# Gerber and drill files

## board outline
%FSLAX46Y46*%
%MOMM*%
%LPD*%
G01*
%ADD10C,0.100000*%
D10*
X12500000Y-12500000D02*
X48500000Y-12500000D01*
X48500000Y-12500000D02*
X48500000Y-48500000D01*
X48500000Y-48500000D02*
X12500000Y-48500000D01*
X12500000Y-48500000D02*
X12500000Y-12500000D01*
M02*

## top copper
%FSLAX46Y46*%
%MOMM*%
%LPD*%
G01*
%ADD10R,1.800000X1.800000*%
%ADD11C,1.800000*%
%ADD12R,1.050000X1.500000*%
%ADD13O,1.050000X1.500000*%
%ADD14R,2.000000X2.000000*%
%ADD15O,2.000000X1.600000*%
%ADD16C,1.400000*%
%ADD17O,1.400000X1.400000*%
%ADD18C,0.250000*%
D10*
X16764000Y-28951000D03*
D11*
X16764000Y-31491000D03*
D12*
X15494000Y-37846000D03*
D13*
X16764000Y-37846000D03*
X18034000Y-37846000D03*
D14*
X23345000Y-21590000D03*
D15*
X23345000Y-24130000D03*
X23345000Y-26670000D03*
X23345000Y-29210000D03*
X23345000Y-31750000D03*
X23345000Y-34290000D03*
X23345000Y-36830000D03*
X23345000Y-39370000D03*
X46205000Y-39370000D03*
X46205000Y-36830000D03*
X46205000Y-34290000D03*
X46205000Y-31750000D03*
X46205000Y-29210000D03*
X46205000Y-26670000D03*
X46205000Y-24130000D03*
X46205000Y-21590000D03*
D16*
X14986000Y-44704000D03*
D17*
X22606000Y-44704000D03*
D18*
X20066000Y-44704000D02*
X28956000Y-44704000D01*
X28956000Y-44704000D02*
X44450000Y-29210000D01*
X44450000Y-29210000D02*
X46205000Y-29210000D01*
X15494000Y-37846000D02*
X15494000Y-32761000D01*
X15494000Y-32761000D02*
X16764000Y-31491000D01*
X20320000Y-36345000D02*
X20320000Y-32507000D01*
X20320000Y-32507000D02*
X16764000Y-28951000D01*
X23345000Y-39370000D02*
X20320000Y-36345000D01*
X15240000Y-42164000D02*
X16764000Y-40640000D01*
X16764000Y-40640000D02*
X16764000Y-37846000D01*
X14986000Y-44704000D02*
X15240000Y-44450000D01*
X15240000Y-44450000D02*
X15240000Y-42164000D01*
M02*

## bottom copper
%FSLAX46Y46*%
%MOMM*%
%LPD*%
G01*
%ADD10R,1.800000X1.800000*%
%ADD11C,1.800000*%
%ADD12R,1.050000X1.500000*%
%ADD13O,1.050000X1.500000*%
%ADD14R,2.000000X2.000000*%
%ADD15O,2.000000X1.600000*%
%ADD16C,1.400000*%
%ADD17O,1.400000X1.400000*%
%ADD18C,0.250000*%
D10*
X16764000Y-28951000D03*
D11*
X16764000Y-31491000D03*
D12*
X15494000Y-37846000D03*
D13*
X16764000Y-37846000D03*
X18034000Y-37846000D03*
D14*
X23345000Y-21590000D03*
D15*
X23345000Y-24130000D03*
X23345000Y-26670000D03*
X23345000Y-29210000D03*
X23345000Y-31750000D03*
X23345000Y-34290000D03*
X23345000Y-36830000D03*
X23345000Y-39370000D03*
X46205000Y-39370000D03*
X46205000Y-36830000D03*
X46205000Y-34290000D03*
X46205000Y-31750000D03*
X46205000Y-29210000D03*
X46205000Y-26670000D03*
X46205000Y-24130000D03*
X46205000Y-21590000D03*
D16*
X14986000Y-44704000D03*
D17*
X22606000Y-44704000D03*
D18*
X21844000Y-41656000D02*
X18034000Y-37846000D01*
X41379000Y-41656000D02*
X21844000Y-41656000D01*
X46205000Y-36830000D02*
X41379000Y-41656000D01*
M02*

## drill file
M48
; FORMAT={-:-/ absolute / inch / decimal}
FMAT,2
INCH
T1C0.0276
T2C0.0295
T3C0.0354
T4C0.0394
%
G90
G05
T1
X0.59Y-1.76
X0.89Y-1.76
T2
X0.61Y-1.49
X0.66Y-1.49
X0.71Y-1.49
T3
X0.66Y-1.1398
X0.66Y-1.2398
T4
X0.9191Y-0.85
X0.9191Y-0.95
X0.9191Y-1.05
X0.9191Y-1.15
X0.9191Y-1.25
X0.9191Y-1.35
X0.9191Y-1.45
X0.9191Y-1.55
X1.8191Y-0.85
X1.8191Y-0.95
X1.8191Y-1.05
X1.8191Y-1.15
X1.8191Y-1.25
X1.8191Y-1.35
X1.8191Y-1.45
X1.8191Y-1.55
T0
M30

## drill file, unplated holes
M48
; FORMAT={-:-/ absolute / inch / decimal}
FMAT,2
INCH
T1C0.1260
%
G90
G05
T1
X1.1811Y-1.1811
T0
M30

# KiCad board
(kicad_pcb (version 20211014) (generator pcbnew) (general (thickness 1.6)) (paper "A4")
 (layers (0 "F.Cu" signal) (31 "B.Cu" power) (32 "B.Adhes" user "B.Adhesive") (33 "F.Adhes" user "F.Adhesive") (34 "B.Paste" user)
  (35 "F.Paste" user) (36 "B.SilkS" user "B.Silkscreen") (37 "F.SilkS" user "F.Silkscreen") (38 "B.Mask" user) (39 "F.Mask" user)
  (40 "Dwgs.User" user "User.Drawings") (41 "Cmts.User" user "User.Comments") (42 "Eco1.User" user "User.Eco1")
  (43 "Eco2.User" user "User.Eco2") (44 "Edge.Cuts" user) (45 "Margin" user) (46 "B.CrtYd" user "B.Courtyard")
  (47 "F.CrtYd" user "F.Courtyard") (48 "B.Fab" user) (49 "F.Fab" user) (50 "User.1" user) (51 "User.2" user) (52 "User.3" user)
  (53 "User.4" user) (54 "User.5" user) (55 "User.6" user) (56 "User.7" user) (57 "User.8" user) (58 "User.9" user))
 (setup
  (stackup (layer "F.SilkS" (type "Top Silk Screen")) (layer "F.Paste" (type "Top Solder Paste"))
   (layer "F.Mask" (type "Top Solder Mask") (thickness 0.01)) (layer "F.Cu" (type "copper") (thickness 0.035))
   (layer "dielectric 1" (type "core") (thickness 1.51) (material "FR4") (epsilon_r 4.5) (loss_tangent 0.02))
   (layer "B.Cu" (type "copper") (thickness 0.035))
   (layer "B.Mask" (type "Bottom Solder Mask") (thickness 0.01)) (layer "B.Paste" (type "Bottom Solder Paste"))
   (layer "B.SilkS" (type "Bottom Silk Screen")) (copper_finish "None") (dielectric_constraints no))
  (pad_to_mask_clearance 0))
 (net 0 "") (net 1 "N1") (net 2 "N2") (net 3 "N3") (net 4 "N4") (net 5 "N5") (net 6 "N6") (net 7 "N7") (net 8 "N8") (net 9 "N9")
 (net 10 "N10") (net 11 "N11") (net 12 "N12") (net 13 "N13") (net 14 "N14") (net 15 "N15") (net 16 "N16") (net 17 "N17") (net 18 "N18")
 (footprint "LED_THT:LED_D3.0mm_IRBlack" (layer "F.Cu") (at 16.764 28.951 -90)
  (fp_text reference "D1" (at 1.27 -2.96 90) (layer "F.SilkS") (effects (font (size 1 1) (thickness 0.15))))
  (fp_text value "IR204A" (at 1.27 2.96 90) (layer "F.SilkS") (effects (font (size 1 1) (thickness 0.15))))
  (pad "1" thru_hole rect (at 0 0 270) (size 1.8 1.8) (drill 0.9) (layers *.Cu *.Mask) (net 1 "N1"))
  (pad "2" thru_hole circle (at 2.54 0 270) (size 1.8 1.8) (drill 0.9) (layers *.Cu *.Mask) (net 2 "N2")))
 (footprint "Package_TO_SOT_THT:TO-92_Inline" (layer "F.Cu") (at 15.494 37.846)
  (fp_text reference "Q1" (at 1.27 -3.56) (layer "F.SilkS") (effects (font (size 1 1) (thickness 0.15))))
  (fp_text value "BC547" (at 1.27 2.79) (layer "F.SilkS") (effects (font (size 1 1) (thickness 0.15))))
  (pad "1" thru_hole rect (at 0 0) (size 1.05 1.5) (drill 0.75) (layers *.Cu *.Mask) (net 2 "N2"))
  (pad "2" thru_hole oval (at 1.27 0) (size 1.05 1.5) (drill 0.75) (layers *.Cu *.Mask) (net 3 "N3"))
  (pad "3" thru_hole oval (at 2.54 0) (size 1.05 1.5) (drill 0.75) (layers *.Cu *.Mask) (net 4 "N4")))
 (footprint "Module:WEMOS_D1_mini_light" (layer "F.Cu") (at 23.345 21.59)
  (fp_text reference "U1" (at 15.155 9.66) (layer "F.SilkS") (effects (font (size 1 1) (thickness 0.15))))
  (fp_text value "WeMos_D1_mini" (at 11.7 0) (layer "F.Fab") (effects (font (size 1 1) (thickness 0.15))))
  (pad "1" thru_hole rect (at 0 0) (size 2 2) (drill 1) (layers *.Cu *.Mask) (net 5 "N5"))
  (pad "2" thru_hole oval (at 0 2.54) (size 2 1.6) (drill 1) (layers *.Cu *.Mask) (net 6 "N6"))
  (pad "3" thru_hole oval (at 0 5.08) (size 2 1.6) (drill 1) (layers *.Cu *.Mask) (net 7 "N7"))
  (pad "4" thru_hole oval (at 0 7.62) (size 2 1.6) (drill 1) (layers *.Cu *.Mask) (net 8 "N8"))
  (pad "5" thru_hole oval (at 0 10.16) (size 2 1.6) (drill 1) (layers *.Cu *.Mask) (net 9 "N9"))
  (pad "6" thru_hole oval (at 0 12.7) (size 2 1.6) (drill 1) (layers *.Cu *.Mask) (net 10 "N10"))
  (pad "7" thru_hole oval (at 0 15.24) (size 2 1.6) (drill 1) (layers *.Cu *.Mask) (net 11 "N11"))
  (pad "8" thru_hole oval (at 0 17.78) (size 2 1.6) (drill 1) (layers *.Cu *.Mask) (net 1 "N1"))
  (pad "9" thru_hole oval (at 22.86 17.78) (size 2 1.6) (drill 1) (layers *.Cu *.Mask) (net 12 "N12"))
  (pad "10" thru_hole oval (at 22.86 15.24) (size 2 1.6) (drill 1) (layers *.Cu *.Mask) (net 4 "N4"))
  (pad "11" thru_hole oval (at 22.86 12.7) (size 2 1.6) (drill 1) (layers *.Cu *.Mask) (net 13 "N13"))
  (pad "12" thru_hole oval (at 22.86 10.16) (size 2 1.6) (drill 1) (layers *.Cu *.Mask) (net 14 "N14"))
  (pad "13" thru_hole oval (at 22.86 7.62) (size 2 1.6) (drill 1) (layers *.Cu *.Mask) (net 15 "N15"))
  (pad "14" thru_hole oval (at 22.86 5.08) (size 2 1.6) (drill 1) (layers *.Cu *.Mask) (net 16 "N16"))
  (pad "15" thru_hole oval (at 22.86 2.54) (size 2 1.6) (drill 1) (layers *.Cu *.Mask) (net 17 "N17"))
  (pad "16" thru_hole oval (at 22.86 0) (size 2 1.6) (drill 1) (layers *.Cu *.Mask) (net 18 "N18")))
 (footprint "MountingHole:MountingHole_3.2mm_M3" (layer "F.Cu") (at 30 30)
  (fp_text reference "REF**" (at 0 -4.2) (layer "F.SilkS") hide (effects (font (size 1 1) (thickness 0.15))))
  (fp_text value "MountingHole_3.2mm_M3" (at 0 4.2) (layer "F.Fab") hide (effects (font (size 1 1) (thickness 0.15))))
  (pad "" np_thru_hole circle (at 0 0) (size 3.2 3.2) (drill 3.2) (layers *.Cu *.Mask)))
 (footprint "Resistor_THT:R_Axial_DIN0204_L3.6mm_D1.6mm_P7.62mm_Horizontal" (layer "F.Cu") (at 14.986 44.704)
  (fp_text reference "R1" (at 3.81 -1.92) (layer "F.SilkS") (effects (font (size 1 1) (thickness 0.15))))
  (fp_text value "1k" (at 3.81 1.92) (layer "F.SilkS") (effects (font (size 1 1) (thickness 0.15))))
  (pad "1" thru_hole circle (at 0 0) (size 1.4 1.4) (drill 0.7) (layers *.Cu *.Mask) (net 3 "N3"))
  (pad "2" thru_hole oval (at 7.62 0) (size 1.4 1.4) (drill 0.7) (layers *.Cu *.Mask) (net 15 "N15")))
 (gr_rect (start 12.5 12.5) (end 48.5 48.5) (layer "Edge.Cuts") (width 0.1) (fill none))
 (segment (start 20.066 44.704) (end 28.956 44.704) (width 0.25) (layer "F.Cu") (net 15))
 (segment (start 28.956 44.704) (end 44.45 29.21) (width 0.25) (layer "F.Cu") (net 15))
 (segment (start 44.45 29.21) (end 46.205 29.21) (width 0.25) (layer "F.Cu") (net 15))
 (segment (start 15.494 37.846) (end 15.494 32.761) (width 0.25) (layer "F.Cu") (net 2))
 (segment (start 15.494 32.761) (end 16.764 31.491) (width 0.25) (layer "F.Cu") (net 2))
 (segment (start 21.844 41.656) (end 18.034 37.846) (width 0.25) (layer "B.Cu") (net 4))
 (segment (start 41.379 41.656) (end 21.844 41.656) (width 0.25) (layer "B.Cu") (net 4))
 (segment (start 46.205 36.83) (end 41.379 41.656) (width 0.25) (layer "B.Cu") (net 4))
 (segment (start 20.32 36.345) (end 20.32 32.507) (width 0.25) (layer "F.Cu") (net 1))
 (segment (start 20.32 32.507) (end 16.764 28.951) (width 0.25) (layer "F.Cu") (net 1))
 (segment (start 23.345 39.37) (end 20.32 36.345) (width 0.25) (layer "F.Cu") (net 1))
 (segment (start 15.24 42.164) (end 16.764 40.64) (width 0.25) (layer "F.Cu") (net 3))
 (segment (start 16.764 40.64) (end 16.764 37.846) (width 0.25) (layer "F.Cu") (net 3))
 (segment (start 14.986 44.704) (end 15.24 44.45) (width 0.25) (layer "F.Cu") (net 3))
 (segment (start 15.24 44.45) (end 15.24 42.164) (width 0.25) (layer "F.Cu") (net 3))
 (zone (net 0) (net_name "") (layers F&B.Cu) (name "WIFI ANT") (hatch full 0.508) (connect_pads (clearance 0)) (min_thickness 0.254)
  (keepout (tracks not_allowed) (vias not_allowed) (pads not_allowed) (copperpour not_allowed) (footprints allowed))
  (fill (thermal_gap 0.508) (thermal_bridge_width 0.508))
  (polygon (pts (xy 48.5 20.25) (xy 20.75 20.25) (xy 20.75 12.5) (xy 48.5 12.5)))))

